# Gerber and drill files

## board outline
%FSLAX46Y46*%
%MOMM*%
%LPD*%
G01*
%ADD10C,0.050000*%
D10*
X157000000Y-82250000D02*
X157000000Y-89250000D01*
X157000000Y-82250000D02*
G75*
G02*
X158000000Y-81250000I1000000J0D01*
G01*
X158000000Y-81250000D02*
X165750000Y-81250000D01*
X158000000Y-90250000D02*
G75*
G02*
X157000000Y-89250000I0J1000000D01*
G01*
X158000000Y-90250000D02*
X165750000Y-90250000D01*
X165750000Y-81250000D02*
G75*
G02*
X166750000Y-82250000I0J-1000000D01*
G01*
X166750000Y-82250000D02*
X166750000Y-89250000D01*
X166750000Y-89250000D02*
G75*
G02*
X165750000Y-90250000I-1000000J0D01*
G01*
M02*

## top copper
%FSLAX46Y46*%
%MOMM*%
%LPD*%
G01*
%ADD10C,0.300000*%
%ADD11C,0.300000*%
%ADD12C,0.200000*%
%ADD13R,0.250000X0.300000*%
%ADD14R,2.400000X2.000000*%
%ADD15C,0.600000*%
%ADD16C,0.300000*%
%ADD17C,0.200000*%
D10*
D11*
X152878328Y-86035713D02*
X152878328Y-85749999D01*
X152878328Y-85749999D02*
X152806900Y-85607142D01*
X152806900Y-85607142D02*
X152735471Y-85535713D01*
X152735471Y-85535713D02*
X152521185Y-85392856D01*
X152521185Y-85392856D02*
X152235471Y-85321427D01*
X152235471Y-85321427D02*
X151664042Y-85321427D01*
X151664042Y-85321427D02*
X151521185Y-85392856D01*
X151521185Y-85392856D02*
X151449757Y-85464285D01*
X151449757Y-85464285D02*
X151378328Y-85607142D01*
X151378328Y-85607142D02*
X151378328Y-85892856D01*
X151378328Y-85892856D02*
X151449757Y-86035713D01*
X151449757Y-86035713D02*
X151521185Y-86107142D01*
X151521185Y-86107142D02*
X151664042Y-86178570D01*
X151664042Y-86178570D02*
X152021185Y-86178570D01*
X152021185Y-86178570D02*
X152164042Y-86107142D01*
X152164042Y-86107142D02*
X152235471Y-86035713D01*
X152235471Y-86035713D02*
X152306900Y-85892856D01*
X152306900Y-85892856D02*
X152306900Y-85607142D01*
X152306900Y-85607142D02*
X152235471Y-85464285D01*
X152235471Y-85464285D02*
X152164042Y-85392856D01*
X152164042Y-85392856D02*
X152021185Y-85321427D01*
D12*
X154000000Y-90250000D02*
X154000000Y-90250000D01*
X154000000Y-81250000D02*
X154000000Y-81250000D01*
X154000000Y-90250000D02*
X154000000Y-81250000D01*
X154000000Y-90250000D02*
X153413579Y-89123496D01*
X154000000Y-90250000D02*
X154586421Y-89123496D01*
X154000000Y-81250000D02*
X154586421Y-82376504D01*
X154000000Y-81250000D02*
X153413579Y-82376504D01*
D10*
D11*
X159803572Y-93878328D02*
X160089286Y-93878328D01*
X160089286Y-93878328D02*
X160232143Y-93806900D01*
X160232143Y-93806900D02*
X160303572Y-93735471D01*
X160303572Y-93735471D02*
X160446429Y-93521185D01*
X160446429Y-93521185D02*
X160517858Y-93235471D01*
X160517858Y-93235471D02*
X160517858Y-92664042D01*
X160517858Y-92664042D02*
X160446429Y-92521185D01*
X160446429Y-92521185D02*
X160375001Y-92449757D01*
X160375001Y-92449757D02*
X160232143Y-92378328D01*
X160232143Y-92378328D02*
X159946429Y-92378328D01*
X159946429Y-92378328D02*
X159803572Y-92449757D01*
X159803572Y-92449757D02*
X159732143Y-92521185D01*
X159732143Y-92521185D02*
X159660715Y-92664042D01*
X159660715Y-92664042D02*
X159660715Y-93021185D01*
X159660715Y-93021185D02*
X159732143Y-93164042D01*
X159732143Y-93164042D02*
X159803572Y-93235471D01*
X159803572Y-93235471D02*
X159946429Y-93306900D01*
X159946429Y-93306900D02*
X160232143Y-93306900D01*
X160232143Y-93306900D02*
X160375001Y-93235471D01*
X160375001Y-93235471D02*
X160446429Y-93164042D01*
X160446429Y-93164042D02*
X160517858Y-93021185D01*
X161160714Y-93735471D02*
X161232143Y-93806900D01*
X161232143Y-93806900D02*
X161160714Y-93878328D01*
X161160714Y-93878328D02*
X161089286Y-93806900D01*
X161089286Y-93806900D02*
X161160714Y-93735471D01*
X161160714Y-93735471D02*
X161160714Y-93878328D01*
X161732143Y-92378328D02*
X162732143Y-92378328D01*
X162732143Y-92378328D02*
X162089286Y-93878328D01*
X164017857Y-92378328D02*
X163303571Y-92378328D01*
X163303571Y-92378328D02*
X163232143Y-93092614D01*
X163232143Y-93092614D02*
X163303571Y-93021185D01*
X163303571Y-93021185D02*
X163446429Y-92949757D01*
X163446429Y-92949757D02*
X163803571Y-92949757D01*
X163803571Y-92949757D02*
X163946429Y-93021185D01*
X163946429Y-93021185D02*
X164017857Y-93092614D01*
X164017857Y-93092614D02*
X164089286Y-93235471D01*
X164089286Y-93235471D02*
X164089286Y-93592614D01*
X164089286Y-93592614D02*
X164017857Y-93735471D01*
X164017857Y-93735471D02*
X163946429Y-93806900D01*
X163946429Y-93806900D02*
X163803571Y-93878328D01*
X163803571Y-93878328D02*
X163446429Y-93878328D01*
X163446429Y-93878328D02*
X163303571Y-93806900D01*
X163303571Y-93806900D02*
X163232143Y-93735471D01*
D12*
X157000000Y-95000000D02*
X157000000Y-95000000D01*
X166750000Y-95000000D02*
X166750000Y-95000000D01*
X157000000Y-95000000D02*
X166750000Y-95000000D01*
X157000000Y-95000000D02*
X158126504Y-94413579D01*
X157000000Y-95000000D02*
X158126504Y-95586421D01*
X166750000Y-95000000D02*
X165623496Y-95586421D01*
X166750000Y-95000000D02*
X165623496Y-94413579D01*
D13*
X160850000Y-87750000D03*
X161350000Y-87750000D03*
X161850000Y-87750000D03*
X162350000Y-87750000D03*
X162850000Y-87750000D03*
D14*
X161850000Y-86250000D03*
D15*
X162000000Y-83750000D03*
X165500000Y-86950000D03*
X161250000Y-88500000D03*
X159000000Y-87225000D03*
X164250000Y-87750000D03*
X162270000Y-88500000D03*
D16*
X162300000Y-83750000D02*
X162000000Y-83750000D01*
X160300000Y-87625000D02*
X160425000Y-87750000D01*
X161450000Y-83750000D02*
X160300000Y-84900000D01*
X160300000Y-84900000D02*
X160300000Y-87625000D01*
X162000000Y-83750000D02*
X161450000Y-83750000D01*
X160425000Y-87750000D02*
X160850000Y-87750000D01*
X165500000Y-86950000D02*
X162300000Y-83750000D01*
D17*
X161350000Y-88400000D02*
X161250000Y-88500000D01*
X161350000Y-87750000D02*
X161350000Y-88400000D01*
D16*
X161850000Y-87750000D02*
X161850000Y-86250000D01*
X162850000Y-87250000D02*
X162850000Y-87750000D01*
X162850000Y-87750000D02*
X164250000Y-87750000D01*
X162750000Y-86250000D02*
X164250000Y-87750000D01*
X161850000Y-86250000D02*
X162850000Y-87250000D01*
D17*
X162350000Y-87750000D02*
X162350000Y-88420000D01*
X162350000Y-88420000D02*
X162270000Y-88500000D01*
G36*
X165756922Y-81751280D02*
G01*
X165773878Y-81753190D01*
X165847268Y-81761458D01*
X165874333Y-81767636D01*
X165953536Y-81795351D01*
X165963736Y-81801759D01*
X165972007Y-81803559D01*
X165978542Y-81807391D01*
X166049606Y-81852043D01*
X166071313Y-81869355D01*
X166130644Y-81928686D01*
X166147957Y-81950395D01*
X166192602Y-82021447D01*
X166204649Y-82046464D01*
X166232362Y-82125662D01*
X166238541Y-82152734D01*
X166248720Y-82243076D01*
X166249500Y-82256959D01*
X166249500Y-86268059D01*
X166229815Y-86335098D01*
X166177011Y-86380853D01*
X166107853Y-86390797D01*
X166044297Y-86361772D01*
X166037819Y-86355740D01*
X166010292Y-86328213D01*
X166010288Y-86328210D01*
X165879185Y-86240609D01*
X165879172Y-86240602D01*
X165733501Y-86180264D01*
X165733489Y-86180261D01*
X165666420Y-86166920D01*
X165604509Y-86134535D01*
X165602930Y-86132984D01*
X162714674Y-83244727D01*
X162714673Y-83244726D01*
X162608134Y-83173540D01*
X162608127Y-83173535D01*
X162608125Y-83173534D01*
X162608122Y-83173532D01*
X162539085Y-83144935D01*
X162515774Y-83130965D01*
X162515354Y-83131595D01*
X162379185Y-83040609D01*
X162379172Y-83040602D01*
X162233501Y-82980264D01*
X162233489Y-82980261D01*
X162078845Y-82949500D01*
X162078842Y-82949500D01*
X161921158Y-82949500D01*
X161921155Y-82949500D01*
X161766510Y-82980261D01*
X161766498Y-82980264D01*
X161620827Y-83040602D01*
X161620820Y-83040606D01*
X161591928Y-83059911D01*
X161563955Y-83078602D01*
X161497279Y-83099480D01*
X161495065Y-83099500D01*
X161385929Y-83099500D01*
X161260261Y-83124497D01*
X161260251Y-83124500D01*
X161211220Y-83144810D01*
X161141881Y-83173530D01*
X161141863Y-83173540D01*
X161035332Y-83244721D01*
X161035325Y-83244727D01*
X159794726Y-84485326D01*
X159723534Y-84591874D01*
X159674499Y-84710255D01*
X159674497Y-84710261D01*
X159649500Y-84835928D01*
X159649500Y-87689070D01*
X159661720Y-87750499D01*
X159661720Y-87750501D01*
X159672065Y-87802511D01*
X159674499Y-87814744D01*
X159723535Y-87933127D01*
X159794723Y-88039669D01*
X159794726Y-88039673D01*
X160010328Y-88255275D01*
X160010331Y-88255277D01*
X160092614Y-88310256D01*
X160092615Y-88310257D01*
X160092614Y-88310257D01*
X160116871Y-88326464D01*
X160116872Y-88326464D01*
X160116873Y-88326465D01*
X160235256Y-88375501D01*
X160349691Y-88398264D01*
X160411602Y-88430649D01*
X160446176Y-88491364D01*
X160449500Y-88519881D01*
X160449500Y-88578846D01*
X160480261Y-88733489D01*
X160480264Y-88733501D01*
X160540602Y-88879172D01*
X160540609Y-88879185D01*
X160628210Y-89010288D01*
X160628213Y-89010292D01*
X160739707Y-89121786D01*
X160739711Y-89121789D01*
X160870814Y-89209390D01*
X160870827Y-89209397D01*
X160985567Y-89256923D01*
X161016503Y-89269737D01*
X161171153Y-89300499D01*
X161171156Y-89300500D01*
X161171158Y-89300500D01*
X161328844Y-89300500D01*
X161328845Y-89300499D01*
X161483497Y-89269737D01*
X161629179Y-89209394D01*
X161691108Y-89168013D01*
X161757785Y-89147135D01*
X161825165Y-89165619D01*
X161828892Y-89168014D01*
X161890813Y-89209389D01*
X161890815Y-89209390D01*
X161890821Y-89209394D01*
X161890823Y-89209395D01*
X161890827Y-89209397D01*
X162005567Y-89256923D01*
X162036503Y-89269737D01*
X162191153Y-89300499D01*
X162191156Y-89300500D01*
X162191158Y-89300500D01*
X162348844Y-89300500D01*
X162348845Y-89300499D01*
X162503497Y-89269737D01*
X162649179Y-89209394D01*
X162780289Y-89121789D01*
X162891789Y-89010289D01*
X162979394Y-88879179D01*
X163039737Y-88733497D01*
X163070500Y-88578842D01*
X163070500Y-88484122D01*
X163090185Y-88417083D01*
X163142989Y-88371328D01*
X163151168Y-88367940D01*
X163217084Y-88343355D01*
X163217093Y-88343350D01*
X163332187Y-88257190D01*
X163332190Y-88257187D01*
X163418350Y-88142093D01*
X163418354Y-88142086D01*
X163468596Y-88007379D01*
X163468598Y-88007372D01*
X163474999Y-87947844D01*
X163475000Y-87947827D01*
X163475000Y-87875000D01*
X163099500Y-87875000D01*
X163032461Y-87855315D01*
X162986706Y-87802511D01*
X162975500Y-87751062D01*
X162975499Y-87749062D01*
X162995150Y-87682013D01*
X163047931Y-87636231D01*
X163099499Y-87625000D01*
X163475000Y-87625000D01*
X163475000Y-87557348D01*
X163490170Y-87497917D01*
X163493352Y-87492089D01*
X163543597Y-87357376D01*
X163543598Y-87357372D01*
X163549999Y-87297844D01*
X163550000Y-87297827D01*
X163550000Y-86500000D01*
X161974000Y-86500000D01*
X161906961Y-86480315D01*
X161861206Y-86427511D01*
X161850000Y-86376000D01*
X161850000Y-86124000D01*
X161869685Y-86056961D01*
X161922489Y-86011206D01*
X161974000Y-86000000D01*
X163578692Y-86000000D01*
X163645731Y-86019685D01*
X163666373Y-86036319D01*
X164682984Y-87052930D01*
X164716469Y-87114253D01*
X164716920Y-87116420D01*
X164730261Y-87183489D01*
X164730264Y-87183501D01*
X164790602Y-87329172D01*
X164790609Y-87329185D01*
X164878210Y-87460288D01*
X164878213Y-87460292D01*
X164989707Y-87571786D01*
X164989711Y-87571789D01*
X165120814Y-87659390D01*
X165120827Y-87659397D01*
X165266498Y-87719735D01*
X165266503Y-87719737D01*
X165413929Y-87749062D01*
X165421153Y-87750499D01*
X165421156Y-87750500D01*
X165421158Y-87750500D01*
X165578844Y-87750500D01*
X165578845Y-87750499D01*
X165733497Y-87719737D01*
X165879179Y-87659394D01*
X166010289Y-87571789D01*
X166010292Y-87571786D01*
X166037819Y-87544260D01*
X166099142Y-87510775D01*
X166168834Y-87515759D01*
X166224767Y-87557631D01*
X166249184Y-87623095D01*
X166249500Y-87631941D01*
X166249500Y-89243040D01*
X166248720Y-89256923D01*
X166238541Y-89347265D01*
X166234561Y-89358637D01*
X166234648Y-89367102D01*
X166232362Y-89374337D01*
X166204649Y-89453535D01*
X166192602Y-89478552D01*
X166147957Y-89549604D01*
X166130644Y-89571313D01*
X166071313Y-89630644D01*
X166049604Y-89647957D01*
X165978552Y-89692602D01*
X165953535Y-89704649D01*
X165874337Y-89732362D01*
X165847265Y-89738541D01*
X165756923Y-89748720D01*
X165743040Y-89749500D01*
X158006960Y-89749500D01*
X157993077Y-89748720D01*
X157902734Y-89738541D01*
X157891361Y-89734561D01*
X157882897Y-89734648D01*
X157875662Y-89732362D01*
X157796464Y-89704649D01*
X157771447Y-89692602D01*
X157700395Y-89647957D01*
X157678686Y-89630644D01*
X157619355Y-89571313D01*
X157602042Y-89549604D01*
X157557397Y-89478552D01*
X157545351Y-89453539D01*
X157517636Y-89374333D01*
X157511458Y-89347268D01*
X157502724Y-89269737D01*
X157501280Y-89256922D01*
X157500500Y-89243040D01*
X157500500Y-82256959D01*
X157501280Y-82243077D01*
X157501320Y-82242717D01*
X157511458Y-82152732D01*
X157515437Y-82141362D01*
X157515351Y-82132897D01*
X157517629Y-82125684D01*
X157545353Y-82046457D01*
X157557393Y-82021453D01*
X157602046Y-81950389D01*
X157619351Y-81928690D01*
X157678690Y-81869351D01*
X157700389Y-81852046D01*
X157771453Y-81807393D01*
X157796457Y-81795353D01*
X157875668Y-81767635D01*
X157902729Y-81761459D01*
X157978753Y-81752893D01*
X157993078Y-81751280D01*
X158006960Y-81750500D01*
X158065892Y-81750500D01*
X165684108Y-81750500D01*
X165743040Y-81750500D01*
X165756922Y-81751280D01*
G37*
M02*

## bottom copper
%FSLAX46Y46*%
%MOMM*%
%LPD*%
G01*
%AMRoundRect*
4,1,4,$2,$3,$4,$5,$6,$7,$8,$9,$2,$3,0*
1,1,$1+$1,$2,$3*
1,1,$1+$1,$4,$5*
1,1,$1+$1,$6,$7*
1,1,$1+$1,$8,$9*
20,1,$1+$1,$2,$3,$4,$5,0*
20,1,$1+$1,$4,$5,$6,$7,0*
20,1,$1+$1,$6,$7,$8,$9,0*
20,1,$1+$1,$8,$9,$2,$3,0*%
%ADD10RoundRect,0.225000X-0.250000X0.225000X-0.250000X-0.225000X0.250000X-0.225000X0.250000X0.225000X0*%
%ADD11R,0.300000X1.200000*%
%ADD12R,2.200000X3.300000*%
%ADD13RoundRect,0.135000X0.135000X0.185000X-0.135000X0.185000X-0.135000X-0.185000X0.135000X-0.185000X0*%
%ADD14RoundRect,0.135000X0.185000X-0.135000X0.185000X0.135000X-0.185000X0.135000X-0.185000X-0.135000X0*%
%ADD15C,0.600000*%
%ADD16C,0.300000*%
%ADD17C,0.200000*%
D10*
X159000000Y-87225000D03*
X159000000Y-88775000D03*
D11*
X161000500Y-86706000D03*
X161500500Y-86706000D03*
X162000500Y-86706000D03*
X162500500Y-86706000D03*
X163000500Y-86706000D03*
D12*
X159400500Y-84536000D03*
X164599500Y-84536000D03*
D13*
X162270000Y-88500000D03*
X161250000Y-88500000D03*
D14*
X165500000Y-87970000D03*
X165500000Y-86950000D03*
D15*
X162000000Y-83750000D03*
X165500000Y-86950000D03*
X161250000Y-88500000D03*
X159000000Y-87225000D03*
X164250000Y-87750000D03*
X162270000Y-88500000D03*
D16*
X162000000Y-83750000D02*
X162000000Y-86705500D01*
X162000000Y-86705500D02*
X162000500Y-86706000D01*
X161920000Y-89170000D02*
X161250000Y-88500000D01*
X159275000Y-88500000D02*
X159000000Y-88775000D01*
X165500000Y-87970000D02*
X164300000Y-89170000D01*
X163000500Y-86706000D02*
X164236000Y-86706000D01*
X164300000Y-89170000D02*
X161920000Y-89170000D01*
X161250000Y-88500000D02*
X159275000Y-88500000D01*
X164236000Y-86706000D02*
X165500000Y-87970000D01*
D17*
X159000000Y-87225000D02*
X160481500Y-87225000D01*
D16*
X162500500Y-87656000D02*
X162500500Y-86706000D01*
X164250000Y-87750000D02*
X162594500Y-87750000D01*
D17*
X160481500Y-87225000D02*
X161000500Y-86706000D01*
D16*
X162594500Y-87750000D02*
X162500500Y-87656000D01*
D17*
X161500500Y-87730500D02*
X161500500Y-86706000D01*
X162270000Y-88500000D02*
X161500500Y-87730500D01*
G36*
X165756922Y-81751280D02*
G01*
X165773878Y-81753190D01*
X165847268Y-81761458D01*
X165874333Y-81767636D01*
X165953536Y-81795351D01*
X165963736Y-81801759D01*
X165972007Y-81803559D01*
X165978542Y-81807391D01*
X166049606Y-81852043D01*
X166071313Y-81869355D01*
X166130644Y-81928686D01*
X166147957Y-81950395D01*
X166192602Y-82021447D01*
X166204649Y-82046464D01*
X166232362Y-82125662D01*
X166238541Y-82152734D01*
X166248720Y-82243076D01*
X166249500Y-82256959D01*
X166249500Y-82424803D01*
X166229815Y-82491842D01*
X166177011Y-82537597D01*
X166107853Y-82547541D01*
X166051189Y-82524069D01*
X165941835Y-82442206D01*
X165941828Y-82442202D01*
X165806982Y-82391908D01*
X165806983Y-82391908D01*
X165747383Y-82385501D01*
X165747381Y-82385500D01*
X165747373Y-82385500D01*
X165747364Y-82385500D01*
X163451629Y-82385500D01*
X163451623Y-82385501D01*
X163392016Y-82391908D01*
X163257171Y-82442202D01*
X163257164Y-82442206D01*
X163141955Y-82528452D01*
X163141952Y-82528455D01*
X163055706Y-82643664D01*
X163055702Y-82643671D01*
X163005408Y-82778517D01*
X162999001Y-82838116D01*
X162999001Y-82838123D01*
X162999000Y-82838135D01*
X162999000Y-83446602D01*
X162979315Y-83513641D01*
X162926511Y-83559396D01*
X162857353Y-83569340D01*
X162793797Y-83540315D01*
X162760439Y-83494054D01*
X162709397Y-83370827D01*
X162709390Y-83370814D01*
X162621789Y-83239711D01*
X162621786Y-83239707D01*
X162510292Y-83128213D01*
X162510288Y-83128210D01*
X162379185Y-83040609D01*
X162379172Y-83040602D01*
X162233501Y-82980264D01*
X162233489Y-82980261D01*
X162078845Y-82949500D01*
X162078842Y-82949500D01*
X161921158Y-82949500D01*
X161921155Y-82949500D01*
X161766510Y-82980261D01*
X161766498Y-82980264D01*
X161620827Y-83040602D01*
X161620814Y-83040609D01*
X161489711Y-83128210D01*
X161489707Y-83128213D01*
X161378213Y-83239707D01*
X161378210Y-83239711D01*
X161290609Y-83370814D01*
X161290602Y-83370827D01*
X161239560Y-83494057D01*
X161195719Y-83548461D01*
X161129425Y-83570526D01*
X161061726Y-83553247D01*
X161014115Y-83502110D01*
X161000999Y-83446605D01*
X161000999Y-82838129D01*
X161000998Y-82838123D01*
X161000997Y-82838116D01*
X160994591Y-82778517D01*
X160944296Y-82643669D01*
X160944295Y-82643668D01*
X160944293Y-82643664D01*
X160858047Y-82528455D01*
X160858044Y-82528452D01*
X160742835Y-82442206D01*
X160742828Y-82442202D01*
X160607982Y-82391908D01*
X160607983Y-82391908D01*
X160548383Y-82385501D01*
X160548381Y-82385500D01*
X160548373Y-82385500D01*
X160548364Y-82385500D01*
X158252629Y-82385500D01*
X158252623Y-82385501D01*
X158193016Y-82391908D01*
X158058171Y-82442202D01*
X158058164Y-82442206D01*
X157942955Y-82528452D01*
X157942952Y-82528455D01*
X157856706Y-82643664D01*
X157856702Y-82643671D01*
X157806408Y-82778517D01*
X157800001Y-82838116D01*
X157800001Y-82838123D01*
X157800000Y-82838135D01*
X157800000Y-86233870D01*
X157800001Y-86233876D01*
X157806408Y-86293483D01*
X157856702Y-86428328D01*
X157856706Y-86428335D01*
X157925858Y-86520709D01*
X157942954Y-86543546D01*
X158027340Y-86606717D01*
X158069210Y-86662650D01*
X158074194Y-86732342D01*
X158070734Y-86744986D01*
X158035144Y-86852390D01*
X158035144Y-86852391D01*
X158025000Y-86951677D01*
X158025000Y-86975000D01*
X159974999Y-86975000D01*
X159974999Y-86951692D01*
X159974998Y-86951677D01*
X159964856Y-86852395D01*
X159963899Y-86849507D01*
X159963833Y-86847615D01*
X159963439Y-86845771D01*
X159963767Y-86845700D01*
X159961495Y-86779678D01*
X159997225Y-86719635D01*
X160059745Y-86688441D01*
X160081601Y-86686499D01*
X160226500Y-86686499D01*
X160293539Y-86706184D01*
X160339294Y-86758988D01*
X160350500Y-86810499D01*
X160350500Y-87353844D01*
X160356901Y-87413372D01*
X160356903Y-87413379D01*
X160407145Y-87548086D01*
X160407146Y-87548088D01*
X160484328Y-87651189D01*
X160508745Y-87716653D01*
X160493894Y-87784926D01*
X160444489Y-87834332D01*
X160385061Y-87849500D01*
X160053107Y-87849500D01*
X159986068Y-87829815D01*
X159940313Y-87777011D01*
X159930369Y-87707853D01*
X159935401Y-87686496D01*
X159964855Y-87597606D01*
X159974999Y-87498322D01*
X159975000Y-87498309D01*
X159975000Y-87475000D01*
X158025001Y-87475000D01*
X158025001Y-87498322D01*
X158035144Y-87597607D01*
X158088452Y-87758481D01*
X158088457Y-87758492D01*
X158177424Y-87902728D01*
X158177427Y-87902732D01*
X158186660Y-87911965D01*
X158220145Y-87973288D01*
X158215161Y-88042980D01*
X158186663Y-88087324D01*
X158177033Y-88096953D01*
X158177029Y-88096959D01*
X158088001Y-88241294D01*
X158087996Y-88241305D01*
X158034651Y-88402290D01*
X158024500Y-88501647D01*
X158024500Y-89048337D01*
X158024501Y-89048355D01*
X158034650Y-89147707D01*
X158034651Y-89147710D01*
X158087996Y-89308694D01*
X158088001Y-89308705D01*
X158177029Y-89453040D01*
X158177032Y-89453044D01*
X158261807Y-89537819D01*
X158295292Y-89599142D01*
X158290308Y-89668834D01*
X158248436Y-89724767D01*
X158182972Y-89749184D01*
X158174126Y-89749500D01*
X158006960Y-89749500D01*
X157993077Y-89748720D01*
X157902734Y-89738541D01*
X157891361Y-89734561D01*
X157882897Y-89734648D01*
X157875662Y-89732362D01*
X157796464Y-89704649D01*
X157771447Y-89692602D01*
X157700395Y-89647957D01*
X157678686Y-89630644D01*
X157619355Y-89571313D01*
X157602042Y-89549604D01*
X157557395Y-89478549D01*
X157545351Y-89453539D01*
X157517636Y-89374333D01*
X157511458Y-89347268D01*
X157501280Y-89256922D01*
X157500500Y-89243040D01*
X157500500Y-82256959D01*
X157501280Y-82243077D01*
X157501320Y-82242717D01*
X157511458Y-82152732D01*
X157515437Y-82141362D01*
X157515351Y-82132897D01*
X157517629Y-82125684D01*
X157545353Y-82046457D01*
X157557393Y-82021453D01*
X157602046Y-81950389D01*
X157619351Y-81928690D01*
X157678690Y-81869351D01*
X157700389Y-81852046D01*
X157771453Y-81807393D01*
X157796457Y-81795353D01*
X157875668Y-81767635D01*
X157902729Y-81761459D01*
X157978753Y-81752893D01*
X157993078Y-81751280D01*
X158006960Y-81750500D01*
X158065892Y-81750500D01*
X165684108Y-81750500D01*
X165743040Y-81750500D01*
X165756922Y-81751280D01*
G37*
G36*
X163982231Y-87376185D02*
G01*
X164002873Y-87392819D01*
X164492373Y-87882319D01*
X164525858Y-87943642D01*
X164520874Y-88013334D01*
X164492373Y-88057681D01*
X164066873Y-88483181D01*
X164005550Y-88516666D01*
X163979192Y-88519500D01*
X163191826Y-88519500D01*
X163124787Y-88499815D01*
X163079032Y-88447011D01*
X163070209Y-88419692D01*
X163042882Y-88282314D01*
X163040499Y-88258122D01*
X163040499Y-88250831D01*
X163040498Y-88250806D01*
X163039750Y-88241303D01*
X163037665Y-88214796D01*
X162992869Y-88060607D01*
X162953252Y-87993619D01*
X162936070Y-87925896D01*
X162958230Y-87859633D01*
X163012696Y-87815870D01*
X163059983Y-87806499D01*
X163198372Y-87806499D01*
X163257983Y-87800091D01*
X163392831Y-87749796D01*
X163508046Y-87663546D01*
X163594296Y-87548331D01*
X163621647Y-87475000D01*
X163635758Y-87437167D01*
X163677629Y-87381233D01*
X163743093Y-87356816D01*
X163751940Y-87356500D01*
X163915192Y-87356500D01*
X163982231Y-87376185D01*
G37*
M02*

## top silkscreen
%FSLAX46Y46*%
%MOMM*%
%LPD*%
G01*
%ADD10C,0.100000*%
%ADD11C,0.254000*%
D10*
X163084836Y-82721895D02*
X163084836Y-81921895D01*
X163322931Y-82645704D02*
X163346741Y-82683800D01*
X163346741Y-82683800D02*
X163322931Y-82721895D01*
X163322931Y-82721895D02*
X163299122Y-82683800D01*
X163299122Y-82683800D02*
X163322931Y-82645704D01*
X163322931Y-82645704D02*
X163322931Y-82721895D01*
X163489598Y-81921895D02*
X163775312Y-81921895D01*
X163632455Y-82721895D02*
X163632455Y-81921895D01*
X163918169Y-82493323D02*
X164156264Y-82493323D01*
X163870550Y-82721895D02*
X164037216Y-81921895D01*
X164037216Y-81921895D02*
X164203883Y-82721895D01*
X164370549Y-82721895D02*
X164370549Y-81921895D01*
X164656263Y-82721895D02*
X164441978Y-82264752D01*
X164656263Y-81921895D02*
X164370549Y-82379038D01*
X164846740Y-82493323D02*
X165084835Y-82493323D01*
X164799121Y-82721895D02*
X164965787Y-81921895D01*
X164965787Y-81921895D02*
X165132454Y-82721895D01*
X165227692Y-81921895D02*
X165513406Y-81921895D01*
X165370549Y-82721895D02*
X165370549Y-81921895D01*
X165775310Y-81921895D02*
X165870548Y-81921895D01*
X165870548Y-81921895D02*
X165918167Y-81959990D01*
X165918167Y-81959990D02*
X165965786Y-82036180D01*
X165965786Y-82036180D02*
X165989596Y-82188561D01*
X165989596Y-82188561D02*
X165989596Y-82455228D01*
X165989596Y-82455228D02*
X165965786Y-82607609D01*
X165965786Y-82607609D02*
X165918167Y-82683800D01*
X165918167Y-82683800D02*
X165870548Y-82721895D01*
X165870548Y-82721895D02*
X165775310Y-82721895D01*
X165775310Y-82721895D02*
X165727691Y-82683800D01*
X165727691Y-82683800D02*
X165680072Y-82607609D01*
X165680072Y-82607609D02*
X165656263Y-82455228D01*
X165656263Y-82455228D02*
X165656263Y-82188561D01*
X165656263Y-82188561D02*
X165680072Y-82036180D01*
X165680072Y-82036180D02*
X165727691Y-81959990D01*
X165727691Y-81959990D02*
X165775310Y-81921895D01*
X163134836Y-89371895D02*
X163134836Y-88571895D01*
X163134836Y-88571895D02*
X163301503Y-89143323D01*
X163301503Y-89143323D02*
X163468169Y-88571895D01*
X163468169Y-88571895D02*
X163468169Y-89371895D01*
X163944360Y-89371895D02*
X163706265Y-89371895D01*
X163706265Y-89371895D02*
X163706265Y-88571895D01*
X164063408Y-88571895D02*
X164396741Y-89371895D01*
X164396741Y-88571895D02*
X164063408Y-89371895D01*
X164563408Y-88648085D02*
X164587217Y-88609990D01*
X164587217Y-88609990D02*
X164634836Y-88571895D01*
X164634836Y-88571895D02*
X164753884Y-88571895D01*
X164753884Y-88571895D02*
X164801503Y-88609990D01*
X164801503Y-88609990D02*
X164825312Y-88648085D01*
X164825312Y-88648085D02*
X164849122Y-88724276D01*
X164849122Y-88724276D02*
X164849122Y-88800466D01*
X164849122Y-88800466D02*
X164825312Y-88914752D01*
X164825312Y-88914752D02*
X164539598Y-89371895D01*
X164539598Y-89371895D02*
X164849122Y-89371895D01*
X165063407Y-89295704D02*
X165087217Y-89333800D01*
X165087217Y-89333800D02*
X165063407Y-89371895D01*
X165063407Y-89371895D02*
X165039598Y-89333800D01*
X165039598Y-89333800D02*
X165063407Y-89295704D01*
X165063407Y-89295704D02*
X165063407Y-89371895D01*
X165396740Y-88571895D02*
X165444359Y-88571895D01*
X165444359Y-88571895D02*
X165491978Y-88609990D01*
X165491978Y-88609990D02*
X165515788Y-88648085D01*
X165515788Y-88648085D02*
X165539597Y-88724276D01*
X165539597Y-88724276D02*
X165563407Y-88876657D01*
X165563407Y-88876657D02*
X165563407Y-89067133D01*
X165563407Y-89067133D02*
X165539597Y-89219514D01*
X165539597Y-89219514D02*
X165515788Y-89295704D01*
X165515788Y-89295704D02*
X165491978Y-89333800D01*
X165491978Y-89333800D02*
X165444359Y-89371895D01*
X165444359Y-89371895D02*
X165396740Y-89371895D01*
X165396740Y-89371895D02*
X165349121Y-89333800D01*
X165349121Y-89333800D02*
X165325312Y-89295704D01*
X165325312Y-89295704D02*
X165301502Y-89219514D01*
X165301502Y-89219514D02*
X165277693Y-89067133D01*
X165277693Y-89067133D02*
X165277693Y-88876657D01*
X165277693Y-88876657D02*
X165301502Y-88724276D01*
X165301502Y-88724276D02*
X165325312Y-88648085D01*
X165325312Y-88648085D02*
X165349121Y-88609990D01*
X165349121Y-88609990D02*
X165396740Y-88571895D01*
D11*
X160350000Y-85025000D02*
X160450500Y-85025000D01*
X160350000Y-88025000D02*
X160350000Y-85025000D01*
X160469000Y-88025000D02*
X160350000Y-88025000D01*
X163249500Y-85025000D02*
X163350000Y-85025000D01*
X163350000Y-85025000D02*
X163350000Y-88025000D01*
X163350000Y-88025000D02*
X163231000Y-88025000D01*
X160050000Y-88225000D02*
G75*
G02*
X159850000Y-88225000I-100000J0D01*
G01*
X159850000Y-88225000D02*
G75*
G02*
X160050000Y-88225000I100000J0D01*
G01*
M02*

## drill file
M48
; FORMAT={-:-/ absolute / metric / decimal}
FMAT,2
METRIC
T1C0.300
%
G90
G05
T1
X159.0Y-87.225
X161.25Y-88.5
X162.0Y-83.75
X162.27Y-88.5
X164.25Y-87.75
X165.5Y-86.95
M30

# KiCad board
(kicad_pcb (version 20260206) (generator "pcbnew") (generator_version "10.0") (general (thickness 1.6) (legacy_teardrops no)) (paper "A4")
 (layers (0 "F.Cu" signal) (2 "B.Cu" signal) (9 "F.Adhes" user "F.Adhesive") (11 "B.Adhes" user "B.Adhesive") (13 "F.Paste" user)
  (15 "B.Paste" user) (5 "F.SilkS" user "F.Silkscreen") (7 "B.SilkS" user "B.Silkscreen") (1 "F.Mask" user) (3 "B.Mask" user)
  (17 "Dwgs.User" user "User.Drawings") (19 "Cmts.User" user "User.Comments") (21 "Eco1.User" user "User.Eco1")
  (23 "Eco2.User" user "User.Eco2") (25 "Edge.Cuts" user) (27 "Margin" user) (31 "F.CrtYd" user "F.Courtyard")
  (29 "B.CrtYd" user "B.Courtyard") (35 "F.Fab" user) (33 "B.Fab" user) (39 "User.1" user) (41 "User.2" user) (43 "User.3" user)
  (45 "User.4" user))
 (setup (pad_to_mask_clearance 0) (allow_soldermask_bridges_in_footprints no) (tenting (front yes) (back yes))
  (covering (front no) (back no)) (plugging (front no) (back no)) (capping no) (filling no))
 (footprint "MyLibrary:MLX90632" (layer "F.Cu") (at 161.85 86.575)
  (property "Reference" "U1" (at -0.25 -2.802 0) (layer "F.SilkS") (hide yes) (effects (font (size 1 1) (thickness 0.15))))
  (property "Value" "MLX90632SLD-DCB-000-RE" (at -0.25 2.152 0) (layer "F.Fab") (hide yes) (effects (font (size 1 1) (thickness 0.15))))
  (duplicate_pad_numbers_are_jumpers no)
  (fp_line (start -1.5 -1.55) (end -1.3995 -1.55) (stroke (width 0.254) (type default)) (layer "F.SilkS"))
  (fp_line (start -1.5 1.45) (end -1.5 -1.55) (stroke (width 0.254) (type default)) (layer "F.SilkS"))
  (fp_line (start -1.381 1.45) (end -1.5 1.45) (stroke (width 0.254) (type default)) (layer "F.SilkS"))
  (fp_line (start 1.3995 -1.55) (end 1.5 -1.55) (stroke (width 0.254) (type default)) (layer "F.SilkS"))
  (fp_line (start 1.5 -1.55) (end 1.5 1.45) (stroke (width 0.254) (type default)) (layer "F.SilkS"))
  (fp_line (start 1.5 1.45) (end 1.381 1.45) (stroke (width 0.254) (type default)) (layer "F.SilkS"))
  (fp_circle (center -1.9 1.65) (end -1.8 1.65) (stroke (width 0.254) (type default)) (fill no) (layer "F.SilkS"))
  (pad "1" smd rect (at -1 1.175) (size 0.25 0.3) (layers "F.Cu" "F.Mask" "F.Paste") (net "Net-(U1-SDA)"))
  (pad "2" smd rect (at -0.5 1.175) (size 0.25 0.3) (layers "F.Cu" "F.Mask" "F.Paste") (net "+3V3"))
  (pad "3" smd rect (at 0 1.175) (size 0.25 0.3) (layers "F.Cu" "F.Mask" "F.Paste") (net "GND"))
  (pad "4" smd rect (at 0.5 1.175) (size 0.25 0.3) (layers "F.Cu" "F.Mask" "F.Paste") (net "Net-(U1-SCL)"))
  (pad "5" smd rect (at 1 1.175) (size 0.25 0.3) (layers "F.Cu" "F.Mask" "F.Paste") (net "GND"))
  (pad "6" smd rect (at 0 -0.325) (size 2.4 2) (layers "F.Cu" "F.Mask" "F.Paste") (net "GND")))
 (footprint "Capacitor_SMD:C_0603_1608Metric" (layer "B.Cu") (at 159 88 -90)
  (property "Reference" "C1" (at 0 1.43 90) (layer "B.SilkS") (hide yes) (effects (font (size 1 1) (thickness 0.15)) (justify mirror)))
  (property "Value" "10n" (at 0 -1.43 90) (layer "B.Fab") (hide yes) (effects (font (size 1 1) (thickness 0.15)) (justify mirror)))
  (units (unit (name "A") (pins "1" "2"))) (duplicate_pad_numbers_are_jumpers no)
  (pad "1" smd roundrect (at -0.775 0 270) (size 0.9 0.95) (layers "B.Cu" "B.Mask" "B.Paste") (roundrect_rratio 0.25) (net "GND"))
  (pad "2" smd roundrect (at 0.775 0 270) (size 0.9 0.95) (layers "B.Cu" "B.Mask" "B.Paste") (roundrect_rratio 0.25) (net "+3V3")))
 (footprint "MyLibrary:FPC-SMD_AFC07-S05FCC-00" (layer "B.Cu") (at 162 85.621)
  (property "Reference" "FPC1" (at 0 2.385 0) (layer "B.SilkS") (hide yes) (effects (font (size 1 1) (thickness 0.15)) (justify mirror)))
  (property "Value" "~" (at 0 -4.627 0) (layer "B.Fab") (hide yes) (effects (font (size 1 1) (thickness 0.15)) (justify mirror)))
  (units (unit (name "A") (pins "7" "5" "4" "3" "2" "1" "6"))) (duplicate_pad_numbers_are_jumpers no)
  (pad "1" smd rect (at -0.9995 1.085) (size 0.3 1.2) (layers "B.Cu" "B.Mask" "B.Paste") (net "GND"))
  (pad "2" smd rect (at -0.4995 1.085) (size 0.3 1.2) (layers "B.Cu" "B.Mask" "B.Paste") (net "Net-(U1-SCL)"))
  (pad "3" smd rect (at 0.0005 1.085) (size 0.3 1.2) (layers "B.Cu" "B.Mask" "B.Paste") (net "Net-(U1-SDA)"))
  (pad "4" smd rect (at 0.5005 1.085) (size 0.3 1.2) (layers "B.Cu" "B.Mask" "B.Paste") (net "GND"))
  (pad "5" smd rect (at 1.0005 1.085) (size 0.3 1.2) (layers "B.Cu" "B.Mask" "B.Paste") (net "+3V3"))
  (pad "6" smd rect (at -2.5995 -1.085) (size 2.2 3.3) (layers "B.Cu" "B.Mask" "B.Paste") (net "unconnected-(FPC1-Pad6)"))
  (pad "7" smd rect (at 2.5995 -1.085) (size 2.2 3.3) (layers "B.Cu" "B.Mask" "B.Paste") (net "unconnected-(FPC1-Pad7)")))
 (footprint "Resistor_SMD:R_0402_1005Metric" (layer "B.Cu") (at 161.76 88.5 180)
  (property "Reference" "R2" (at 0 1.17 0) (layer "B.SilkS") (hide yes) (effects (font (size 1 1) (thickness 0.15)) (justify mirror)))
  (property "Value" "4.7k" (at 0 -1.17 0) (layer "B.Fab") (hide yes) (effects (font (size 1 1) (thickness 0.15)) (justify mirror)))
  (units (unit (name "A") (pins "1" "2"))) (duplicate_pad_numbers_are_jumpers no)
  (pad "1" smd roundrect (at -0.51 0 180) (size 0.54 0.64) (layers "B.Cu" "B.Mask" "B.Paste") (roundrect_rratio 0.25) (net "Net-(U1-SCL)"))
  (pad "2" smd roundrect (at 0.51 0 180) (size 0.54 0.64) (layers "B.Cu" "B.Mask" "B.Paste") (roundrect_rratio 0.25) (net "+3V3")))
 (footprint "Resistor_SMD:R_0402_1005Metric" (layer "B.Cu") (at 165.5 87.46 90)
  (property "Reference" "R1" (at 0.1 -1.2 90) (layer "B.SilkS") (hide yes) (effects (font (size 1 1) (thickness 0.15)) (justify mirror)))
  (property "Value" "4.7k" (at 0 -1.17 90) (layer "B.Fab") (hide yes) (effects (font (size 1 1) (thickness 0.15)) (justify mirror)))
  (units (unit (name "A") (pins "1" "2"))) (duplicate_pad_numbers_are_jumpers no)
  (pad "1" smd roundrect (at -0.51 0 90) (size 0.54 0.64) (layers "B.Cu" "B.Mask" "B.Paste") (roundrect_rratio 0.25) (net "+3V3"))
  (pad "2" smd roundrect (at 0.51 0 90) (size 0.54 0.64) (layers "B.Cu" "B.Mask" "B.Paste") (roundrect_rratio 0.25) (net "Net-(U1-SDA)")))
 (gr_line (start 157 82.25) (end 157 89.25) (stroke (width 0.05) (type default)) (layer "Edge.Cuts"))
 (gr_arc (start 157 82.25) (mid 157.292893 81.542893) (end 158 81.25) (stroke (width 0.05) (type default)) (layer "Edge.Cuts"))
 (gr_line (start 158 81.25) (end 165.75 81.25) (stroke (width 0.05) (type default)) (layer "Edge.Cuts"))
 (gr_arc (start 158 90.25) (mid 157.292893 89.957107) (end 157 89.25) (stroke (width 0.05) (type default)) (layer "Edge.Cuts"))
 (gr_line (start 158 90.25) (end 165.75 90.25) (stroke (width 0.05) (type default)) (layer "Edge.Cuts"))
 (gr_arc (start 165.75 81.25) (mid 166.457107 81.542893) (end 166.75 82.25) (stroke (width 0.05) (type default)) (layer "Edge.Cuts"))
 (gr_line (start 166.75 82.25) (end 166.75 89.25) (stroke (width 0.05) (type default)) (layer "Edge.Cuts"))
 (gr_arc (start 166.75 89.25) (mid 166.457107 89.957107) (end 165.75 90.25) (stroke (width 0.05) (type default)) (layer "Edge.Cuts"))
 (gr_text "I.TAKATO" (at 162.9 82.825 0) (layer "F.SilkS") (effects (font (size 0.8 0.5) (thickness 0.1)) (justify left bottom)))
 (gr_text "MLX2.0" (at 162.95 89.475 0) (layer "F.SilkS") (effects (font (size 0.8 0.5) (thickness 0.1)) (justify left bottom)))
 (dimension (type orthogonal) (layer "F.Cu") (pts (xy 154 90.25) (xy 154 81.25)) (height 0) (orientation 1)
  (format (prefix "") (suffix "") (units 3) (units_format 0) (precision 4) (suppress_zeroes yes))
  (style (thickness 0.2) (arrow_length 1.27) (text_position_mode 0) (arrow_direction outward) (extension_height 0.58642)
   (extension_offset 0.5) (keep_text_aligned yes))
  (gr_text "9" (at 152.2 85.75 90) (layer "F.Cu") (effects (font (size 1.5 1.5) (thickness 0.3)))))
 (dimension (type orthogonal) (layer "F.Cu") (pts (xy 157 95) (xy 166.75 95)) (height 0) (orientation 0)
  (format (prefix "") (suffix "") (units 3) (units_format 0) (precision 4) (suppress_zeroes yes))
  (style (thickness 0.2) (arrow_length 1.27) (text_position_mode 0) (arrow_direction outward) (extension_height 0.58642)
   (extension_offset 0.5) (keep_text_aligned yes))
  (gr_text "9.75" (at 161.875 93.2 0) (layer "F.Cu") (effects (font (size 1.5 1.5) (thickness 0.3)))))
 (segment (start 162.3 83.75) (end 162 83.75) (width 0.3) (layer "F.Cu") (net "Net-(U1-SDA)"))
 (segment (start 160.3 87.625) (end 160.425 87.75) (width 0.3) (layer "F.Cu") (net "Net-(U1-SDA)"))
 (segment (start 161.45 83.75) (end 160.3 84.9) (width 0.3) (layer "F.Cu") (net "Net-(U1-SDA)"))
 (segment (start 160.3 84.9) (end 160.3 87.625) (width 0.3) (layer "F.Cu") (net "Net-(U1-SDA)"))
 (segment (start 162 83.75) (end 161.45 83.75) (width 0.3) (layer "F.Cu") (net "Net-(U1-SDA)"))
 (segment (start 160.425 87.75) (end 160.85 87.75) (width 0.3) (layer "F.Cu") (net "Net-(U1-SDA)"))
 (segment (start 165.5 86.95) (end 162.3 83.75) (width 0.3) (layer "F.Cu") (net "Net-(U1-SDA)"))
 (via (at 162 83.75) (size 0.6) (drill 0.3) (layers "F.Cu" "B.Cu") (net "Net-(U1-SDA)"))
 (via (at 165.5 86.95) (size 0.6) (drill 0.3) (layers "F.Cu" "B.Cu") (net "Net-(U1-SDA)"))
 (segment (start 162 83.75) (end 162 86.7055) (width 0.3) (layer "B.Cu") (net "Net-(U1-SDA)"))
 (segment (start 162 86.7055) (end 162.0005 86.706) (width 0.3) (layer "B.Cu") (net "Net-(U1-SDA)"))
 (segment (start 161.35 88.4) (end 161.25 88.5) (width 0.2) (layer "F.Cu") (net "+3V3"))
 (segment (start 161.35 87.75) (end 161.35 88.4) (width 0.2) (layer "F.Cu") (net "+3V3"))
 (via (at 161.25 88.5) (size 0.6) (drill 0.3) (layers "F.Cu" "B.Cu") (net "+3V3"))
 (segment (start 161.92 89.17) (end 161.25 88.5) (width 0.3) (layer "B.Cu") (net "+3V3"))
 (segment (start 159.275 88.5) (end 159 88.775) (width 0.3) (layer "B.Cu") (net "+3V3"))
 (segment (start 165.5 87.97) (end 164.3 89.17) (width 0.3) (layer "B.Cu") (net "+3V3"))
 (segment (start 163.0005 86.706) (end 164.236 86.706) (width 0.3) (layer "B.Cu") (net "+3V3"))
 (segment (start 164.3 89.17) (end 161.92 89.17) (width 0.3) (layer "B.Cu") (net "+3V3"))
 (segment (start 161.25 88.5) (end 159.275 88.5) (width 0.3) (layer "B.Cu") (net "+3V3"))
 (segment (start 164.236 86.706) (end 165.5 87.97) (width 0.3) (layer "B.Cu") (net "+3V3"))
 (segment (start 161.85 87.75) (end 161.85 86.25) (width 0.3) (layer "F.Cu") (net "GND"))
 (segment (start 162.85 87.25) (end 162.85 87.75) (width 0.3) (layer "F.Cu") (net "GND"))
 (segment (start 162.85 87.75) (end 164.25 87.75) (width 0.3) (layer "F.Cu") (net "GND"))
 (segment (start 162.75 86.25) (end 164.25 87.75) (width 0.3) (layer "F.Cu") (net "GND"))
 (segment (start 161.85 86.25) (end 162.85 87.25) (width 0.3) (layer "F.Cu") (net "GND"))
 (via (at 159 87.225) (size 0.6) (drill 0.3) (layers "F.Cu" "B.Cu") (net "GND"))
 (via (at 164.25 87.75) (size 0.6) (drill 0.3) (layers "F.Cu" "B.Cu") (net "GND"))
 (segment (start 159 87.225) (end 160.4815 87.225) (width 0.2) (layer "B.Cu") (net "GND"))
 (segment (start 162.5005 87.656) (end 162.5005 86.706) (width 0.3) (layer "B.Cu") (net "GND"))
 (segment (start 164.25 87.75) (end 162.5945 87.75) (width 0.3) (layer "B.Cu") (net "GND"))
 (segment (start 160.4815 87.225) (end 161.0005 86.706) (width 0.2) (layer "B.Cu") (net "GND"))
 (segment (start 162.5945 87.75) (end 162.5005 87.656) (width 0.3) (layer "B.Cu") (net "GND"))
 (segment (start 162.35 87.75) (end 162.35 88.42) (width 0.2) (layer "F.Cu") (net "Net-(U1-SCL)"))
 (segment (start 162.35 88.42) (end 162.27 88.5) (width 0.2) (layer "F.Cu") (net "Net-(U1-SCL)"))
 (via (at 162.27 88.5) (size 0.6) (drill 0.3) (layers "F.Cu" "B.Cu") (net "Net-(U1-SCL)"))
 (segment (start 161.5005 87.7305) (end 161.5005 86.706) (width 0.2) (layer "B.Cu") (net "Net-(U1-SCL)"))
 (segment (start 162.27 88.5) (end 161.5005 87.7305) (width 0.2) (layer "B.Cu") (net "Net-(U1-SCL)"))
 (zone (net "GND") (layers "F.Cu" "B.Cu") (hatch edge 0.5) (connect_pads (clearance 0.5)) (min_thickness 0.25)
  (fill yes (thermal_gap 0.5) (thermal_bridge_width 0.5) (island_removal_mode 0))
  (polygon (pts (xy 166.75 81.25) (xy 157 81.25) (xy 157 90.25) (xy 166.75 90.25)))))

